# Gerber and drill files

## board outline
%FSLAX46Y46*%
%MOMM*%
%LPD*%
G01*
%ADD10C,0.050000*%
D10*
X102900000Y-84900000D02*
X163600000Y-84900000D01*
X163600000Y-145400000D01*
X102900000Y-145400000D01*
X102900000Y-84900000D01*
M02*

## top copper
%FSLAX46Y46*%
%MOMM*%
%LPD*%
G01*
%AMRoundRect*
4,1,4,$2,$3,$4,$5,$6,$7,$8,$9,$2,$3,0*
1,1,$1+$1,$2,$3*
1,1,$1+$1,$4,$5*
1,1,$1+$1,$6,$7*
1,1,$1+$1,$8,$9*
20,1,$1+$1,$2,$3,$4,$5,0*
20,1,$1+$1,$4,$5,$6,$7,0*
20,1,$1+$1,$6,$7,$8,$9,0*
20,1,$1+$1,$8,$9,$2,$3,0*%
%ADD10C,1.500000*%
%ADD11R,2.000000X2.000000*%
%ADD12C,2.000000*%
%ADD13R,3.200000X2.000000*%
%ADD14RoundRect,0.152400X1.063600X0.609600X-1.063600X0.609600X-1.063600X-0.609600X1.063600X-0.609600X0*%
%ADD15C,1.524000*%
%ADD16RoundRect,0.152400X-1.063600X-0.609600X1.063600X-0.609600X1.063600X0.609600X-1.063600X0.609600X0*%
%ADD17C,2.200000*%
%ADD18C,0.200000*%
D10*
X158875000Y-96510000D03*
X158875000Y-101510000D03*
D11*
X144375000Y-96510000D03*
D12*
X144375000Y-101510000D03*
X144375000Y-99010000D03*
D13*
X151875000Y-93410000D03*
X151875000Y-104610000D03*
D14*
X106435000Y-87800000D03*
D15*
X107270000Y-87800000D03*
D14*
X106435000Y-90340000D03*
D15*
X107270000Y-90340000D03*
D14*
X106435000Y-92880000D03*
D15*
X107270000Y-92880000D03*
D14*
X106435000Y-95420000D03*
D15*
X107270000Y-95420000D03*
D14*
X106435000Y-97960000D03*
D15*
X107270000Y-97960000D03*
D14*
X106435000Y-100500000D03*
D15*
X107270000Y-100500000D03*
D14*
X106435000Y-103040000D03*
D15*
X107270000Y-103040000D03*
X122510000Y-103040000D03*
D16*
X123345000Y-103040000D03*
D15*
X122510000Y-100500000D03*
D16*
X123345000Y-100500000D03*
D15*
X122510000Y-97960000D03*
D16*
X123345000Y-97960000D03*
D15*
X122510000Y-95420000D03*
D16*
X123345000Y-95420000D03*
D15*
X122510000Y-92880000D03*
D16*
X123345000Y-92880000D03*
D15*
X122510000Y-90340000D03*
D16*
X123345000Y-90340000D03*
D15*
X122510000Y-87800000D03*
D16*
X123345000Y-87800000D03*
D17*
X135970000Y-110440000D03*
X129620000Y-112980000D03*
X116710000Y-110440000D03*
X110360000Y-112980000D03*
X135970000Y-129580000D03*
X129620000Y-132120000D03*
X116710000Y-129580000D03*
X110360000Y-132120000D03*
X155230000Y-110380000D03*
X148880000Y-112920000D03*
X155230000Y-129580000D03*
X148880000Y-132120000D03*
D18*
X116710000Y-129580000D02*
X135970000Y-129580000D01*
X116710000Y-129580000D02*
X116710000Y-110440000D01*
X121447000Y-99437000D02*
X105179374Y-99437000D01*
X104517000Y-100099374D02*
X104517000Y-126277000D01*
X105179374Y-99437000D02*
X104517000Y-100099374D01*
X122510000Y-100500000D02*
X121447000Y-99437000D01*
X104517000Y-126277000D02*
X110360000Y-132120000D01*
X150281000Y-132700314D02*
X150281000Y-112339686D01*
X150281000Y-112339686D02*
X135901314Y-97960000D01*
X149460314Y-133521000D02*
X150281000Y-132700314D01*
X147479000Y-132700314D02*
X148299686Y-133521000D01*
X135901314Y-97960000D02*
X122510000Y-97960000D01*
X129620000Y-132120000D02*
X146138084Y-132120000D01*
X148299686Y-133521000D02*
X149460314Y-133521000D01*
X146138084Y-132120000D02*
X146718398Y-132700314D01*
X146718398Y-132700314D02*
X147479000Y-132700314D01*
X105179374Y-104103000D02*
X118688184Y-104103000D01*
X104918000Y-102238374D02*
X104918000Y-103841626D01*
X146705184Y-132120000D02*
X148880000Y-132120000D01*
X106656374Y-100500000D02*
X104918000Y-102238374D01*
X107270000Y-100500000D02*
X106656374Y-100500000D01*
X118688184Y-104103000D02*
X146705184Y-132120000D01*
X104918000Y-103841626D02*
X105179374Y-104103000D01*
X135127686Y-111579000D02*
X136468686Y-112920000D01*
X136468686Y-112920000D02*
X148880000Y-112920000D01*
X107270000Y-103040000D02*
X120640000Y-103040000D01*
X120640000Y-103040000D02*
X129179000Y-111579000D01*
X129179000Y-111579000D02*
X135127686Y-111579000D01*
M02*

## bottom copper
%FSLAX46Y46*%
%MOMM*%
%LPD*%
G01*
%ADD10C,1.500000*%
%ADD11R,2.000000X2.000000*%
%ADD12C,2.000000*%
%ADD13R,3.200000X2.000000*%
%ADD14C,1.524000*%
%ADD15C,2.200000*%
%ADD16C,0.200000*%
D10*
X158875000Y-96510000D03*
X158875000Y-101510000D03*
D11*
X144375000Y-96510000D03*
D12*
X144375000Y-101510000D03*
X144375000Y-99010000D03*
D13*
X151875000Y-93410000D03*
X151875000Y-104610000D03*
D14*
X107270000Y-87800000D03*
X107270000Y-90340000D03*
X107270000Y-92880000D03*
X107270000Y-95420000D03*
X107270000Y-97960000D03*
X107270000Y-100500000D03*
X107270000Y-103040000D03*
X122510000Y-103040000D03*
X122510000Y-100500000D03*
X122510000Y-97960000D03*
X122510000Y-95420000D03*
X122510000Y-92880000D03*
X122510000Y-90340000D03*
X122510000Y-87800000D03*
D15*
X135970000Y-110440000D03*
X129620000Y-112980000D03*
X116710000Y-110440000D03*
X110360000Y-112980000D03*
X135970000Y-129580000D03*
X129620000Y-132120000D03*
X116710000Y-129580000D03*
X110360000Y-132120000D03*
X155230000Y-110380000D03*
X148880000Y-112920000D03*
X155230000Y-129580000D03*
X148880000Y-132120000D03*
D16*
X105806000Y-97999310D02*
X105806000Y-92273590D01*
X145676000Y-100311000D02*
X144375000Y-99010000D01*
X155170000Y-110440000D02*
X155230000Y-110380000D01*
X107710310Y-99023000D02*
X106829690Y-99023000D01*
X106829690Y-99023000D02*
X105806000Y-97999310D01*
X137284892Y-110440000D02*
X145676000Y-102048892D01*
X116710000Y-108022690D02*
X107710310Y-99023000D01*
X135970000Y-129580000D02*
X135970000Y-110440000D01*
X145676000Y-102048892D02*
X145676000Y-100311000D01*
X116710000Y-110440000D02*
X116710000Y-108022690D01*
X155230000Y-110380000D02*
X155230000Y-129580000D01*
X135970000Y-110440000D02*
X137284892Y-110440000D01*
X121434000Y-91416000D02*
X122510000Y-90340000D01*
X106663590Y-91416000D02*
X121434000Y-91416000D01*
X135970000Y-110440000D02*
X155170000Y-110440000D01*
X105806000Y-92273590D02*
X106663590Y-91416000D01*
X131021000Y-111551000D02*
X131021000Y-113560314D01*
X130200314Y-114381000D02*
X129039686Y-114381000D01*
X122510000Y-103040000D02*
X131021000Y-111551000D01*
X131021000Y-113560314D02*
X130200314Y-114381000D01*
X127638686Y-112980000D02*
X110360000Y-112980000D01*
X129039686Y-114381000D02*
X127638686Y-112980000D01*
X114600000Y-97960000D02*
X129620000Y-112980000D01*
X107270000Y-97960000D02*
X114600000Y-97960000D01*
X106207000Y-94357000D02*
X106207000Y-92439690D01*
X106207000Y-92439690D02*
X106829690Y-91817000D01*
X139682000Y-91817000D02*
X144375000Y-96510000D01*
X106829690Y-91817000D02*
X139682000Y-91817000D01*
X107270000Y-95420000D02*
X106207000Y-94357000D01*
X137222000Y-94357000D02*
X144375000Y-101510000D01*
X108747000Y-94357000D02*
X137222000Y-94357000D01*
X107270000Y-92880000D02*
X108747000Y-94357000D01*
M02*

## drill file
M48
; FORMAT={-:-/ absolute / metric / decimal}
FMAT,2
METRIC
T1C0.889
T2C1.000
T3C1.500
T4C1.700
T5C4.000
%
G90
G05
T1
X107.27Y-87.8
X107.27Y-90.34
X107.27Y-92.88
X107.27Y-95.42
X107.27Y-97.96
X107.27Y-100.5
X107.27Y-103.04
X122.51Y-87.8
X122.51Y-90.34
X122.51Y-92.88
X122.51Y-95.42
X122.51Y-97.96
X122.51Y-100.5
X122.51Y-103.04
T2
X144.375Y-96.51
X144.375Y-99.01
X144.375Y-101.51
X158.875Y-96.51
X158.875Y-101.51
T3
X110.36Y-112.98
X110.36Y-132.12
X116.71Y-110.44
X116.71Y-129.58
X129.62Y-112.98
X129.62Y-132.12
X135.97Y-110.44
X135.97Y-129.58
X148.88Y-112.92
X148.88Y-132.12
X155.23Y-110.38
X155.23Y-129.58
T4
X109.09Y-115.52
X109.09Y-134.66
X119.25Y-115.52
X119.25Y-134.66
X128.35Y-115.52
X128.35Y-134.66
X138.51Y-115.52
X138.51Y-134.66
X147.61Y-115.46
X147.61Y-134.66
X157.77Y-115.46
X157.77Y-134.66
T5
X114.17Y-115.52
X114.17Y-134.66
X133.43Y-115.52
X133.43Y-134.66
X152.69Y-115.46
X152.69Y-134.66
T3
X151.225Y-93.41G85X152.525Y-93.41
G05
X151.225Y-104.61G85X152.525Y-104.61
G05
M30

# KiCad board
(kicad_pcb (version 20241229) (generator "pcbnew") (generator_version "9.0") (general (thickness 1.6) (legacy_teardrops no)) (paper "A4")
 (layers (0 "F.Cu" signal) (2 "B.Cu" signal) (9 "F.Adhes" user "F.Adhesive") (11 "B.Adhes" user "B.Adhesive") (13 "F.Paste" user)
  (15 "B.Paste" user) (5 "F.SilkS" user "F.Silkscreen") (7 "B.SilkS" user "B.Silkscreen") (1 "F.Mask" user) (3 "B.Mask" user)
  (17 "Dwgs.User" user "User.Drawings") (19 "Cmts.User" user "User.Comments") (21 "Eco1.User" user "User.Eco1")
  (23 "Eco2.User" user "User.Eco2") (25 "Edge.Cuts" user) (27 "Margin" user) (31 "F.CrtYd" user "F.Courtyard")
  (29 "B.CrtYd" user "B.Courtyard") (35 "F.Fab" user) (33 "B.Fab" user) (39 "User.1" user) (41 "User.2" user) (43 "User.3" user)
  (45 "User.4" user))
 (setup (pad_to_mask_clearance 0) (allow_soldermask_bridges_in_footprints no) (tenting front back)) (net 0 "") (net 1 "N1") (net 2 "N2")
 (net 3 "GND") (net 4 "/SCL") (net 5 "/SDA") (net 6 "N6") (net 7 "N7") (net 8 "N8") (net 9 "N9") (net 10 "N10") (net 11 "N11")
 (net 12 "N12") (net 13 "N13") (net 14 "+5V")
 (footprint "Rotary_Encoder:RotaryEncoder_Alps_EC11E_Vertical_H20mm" (layer "F.Cu") (at 144.375 96.51)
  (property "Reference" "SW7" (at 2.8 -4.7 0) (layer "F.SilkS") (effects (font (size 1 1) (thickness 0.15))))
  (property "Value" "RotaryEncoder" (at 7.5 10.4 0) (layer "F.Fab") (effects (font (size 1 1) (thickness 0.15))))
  (pad "" thru_hole circle (at 14.5 0) (size 1.5 1.5) (drill 1) (layers "*.Cu" "*.Mask") (remove_unused_layers no))
  (pad "" thru_hole circle (at 14.5 5) (size 1.5 1.5) (drill 1) (layers "*.Cu" "*.Mask") (remove_unused_layers no))
  (pad "A" thru_hole rect (at 0 0) (size 2 2) (drill 1) (layers "*.Cu" "*.Mask") (remove_unused_layers no) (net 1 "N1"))
  (pad "B" thru_hole circle (at 0 5) (size 2 2) (drill 1) (layers "*.Cu" "*.Mask") (remove_unused_layers no) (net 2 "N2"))
  (pad "C" thru_hole circle (at 0 2.5) (size 2 2) (drill 1) (layers "*.Cu" "*.Mask") (remove_unused_layers no) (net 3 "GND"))
  (pad "MP" thru_hole rect (at 7.5 -3.1) (size 3.2 2) (drill oval 2.8 1.5) (layers "*.Cu" "*.Mask") (remove_unused_layers no))
  (pad "MP" thru_hole rect (at 7.5 8.1) (size 3.2 2) (drill oval 2.8 1.5) (layers "*.Cu" "*.Mask") (remove_unused_layers no)))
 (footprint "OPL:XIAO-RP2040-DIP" (layer "F.Cu") (at 114.89 95.42)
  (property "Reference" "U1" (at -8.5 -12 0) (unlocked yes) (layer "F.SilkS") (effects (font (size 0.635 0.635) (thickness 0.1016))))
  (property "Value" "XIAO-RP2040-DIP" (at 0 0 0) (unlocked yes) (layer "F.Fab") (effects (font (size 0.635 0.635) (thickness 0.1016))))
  (pad "1" smd roundrect (at -8.455 -7.62 180) (size 2.432 1.524) (layers "F.Cu" "F.Mask") (roundrect_rratio 0.1) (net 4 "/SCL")
   (thermal_bridge_angle 45))
  (pad "1" thru_hole circle (at -7.62 -7.62 180) (size 1.524 1.524) (drill 0.889) (layers "*.Cu" "*.Mask") (remove_unused_layers no)
   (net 4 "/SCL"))
  (pad "2" smd roundrect (at -8.455 -5.08 180) (size 2.432 1.524) (layers "F.Cu" "F.Mask") (roundrect_rratio 0.1) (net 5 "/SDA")
   (thermal_bridge_angle 45))
  (pad "2" thru_hole circle (at -7.62 -5.08 180) (size 1.524 1.524) (drill 0.889) (layers "*.Cu" "*.Mask") (remove_unused_layers no)
   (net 5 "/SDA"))
  (pad "3" smd roundrect (at -8.455 -2.54 180) (size 2.432 1.524) (layers "F.Cu" "F.Mask") (roundrect_rratio 0.1) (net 2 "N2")
   (thermal_bridge_angle 45))
  (pad "3" thru_hole circle (at -7.62 -2.54 180) (size 1.524 1.524) (drill 0.889) (layers "*.Cu" "*.Mask") (remove_unused_layers no)
   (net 2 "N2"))
  (pad "4" smd roundrect (at -8.455 0 180) (size 2.432 1.524) (layers "F.Cu" "F.Mask") (roundrect_rratio 0.1) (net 1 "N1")
   (thermal_bridge_angle 45))
  (pad "4" thru_hole circle (at -7.62 0 180) (size 1.524 1.524) (drill 0.889) (layers "*.Cu" "*.Mask") (remove_unused_layers no)
   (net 1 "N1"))
  (pad "5" smd roundrect (at -8.455 2.54 180) (size 2.432 1.524) (layers "F.Cu" "F.Mask") (roundrect_rratio 0.1) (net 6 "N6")
   (thermal_bridge_angle 45))
  (pad "5" thru_hole circle (at -7.62 2.54 180) (size 1.524 1.524) (drill 0.889) (layers "*.Cu" "*.Mask") (remove_unused_layers no)
   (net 6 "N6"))
  (pad "6" smd roundrect (at -8.455 5.08 180) (size 2.432 1.524) (layers "F.Cu" "F.Mask") (roundrect_rratio 0.1) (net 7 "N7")
   (thermal_bridge_angle 45))
  (pad "6" thru_hole circle (at -7.62 5.08 180) (size 1.524 1.524) (drill 0.889) (layers "*.Cu" "*.Mask") (remove_unused_layers no)
   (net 7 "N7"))
  (pad "7" smd roundrect (at -8.455 7.62 180) (size 2.432 1.524) (layers "F.Cu" "F.Mask") (roundrect_rratio 0.1) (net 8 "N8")
   (thermal_bridge_angle 45))
  (pad "7" thru_hole circle (at -7.62 7.62 180) (size 1.524 1.524) (drill 0.889) (layers "*.Cu" "*.Mask") (remove_unused_layers no)
   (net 8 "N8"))
  (pad "8" thru_hole circle (at 7.62 7.62) (size 1.524 1.524) (drill 0.889) (layers "*.Cu" "*.Mask") (remove_unused_layers no) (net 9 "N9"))
  (pad "8" smd roundrect (at 8.455 7.62) (size 2.432 1.524) (layers "F.Cu" "F.Mask") (roundrect_rratio 0.1) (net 9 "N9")
   (thermal_bridge_angle 45))
  (pad "9" thru_hole circle (at 7.62 5.08) (size 1.524 1.524) (drill 0.889) (layers "*.Cu" "*.Mask") (remove_unused_layers no)
   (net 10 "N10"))
  (pad "9" smd roundrect (at 8.455 5.08) (size 2.432 1.524) (layers "F.Cu" "F.Mask") (roundrect_rratio 0.1) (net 10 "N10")
   (thermal_bridge_angle 45))
  (pad "10" thru_hole circle (at 7.62 2.54) (size 1.524 1.524) (drill 0.889) (layers "*.Cu" "*.Mask") (remove_unused_layers no)
   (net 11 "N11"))
  (pad "10" smd roundrect (at 8.455 2.54) (size 2.432 1.524) (layers "F.Cu" "F.Mask") (roundrect_rratio 0.1) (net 11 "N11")
   (thermal_bridge_angle 45))
  (pad "11" thru_hole circle (at 7.62 0) (size 1.524 1.524) (drill 0.889) (layers "*.Cu" "*.Mask") (remove_unused_layers no) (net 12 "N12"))
  (pad "11" smd roundrect (at 8.455 0) (size 2.432 1.524) (layers "F.Cu" "F.Mask") (roundrect_rratio 0.1) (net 12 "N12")
   (thermal_bridge_angle 45))
  (pad "12" thru_hole circle (at 7.62 -2.54) (size 1.524 1.524) (drill 0.889) (layers "*.Cu" "*.Mask") (remove_unused_layers no)
   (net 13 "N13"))
  (pad "12" smd roundrect (at 8.455 -2.54) (size 2.432 1.524) (layers "F.Cu" "F.Mask") (roundrect_rratio 0.1) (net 13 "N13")
   (thermal_bridge_angle 45))
  (pad "13" thru_hole circle (at 7.62 -5.08) (size 1.524 1.524) (drill 0.889) (layers "*.Cu" "*.Mask") (remove_unused_layers no)
   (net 3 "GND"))
  (pad "13" smd roundrect (at 8.455 -5.08) (size 2.432 1.524) (layers "F.Cu" "F.Mask") (roundrect_rratio 0.1) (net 3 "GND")
   (thermal_bridge_angle 45))
  (pad "14" thru_hole circle (at 7.62 -7.62) (size 1.524 1.524) (drill 0.889) (layers "*.Cu" "*.Mask") (remove_unused_layers no)
   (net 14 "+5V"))
  (pad "14" smd roundrect (at 8.455 -7.62) (size 2.432 1.524) (layers "F.Cu" "F.Mask") (roundrect_rratio 0.1) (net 14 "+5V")
   (thermal_bridge_angle 45)))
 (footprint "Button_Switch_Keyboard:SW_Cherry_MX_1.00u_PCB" (layer "F.Cu") (at 135.97 110.44)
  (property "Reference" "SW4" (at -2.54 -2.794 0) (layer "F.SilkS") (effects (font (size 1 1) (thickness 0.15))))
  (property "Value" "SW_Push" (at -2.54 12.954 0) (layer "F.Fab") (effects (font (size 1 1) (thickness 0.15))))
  (pad "" np_thru_hole circle (at -7.62 5.08) (size 1.7 1.7) (drill 1.7) (layers "*.Cu" "*.Mask"))
  (pad "" np_thru_hole circle (at -2.54 5.08) (size 4 4) (drill 4) (layers "*.Cu" "*.Mask"))
  (pad "" np_thru_hole circle (at 2.54 5.08) (size 1.7 1.7) (drill 1.7) (layers "*.Cu" "*.Mask"))
  (pad "1" thru_hole circle (at 0 0) (size 2.2 2.2) (drill 1.5) (layers "*.Cu" "*.Mask") (remove_unused_layers no) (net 3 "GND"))
  (pad "2" thru_hole circle (at -6.35 2.54) (size 2.2 2.2) (drill 1.5) (layers "*.Cu" "*.Mask") (remove_unused_layers no) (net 6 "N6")))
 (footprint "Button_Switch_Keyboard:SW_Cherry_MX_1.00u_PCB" (layer "F.Cu") (at 116.71 110.44)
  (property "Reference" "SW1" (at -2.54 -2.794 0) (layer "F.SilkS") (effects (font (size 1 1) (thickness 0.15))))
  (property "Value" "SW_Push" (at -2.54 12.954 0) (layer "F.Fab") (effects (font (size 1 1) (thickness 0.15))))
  (pad "" np_thru_hole circle (at -7.62 5.08) (size 1.7 1.7) (drill 1.7) (layers "*.Cu" "*.Mask"))
  (pad "" np_thru_hole circle (at -2.54 5.08) (size 4 4) (drill 4) (layers "*.Cu" "*.Mask"))
  (pad "" np_thru_hole circle (at 2.54 5.08) (size 1.7 1.7) (drill 1.7) (layers "*.Cu" "*.Mask"))
  (pad "1" thru_hole circle (at 0 0) (size 2.2 2.2) (drill 1.5) (layers "*.Cu" "*.Mask") (remove_unused_layers no) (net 3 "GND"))
  (pad "2" thru_hole circle (at -6.35 2.54) (size 2.2 2.2) (drill 1.5) (layers "*.Cu" "*.Mask") (remove_unused_layers no) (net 9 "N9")))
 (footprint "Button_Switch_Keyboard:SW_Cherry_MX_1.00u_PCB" (layer "F.Cu") (at 135.97 129.58)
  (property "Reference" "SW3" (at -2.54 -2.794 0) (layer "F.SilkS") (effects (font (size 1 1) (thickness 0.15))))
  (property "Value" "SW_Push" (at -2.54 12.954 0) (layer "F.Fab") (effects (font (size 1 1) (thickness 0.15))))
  (pad "" np_thru_hole circle (at -7.62 5.08) (size 1.7 1.7) (drill 1.7) (layers "*.Cu" "*.Mask"))
  (pad "" np_thru_hole circle (at -2.54 5.08) (size 4 4) (drill 4) (layers "*.Cu" "*.Mask"))
  (pad "" np_thru_hole circle (at 2.54 5.08) (size 1.7 1.7) (drill 1.7) (layers "*.Cu" "*.Mask"))
  (pad "1" thru_hole circle (at 0 0) (size 2.2 2.2) (drill 1.5) (layers "*.Cu" "*.Mask") (remove_unused_layers no) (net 3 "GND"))
  (pad "2" thru_hole circle (at -6.35 2.54) (size 2.2 2.2) (drill 1.5) (layers "*.Cu" "*.Mask") (remove_unused_layers no) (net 11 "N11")))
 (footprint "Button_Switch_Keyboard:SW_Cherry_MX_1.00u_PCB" (layer "F.Cu") (at 116.71 129.58)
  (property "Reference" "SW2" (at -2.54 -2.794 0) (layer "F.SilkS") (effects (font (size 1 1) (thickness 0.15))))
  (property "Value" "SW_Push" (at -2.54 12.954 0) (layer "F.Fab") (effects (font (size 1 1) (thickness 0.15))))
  (pad "" np_thru_hole circle (at -7.62 5.08) (size 1.7 1.7) (drill 1.7) (layers "*.Cu" "*.Mask"))
  (pad "" np_thru_hole circle (at -2.54 5.08) (size 4 4) (drill 4) (layers "*.Cu" "*.Mask"))
  (pad "" np_thru_hole circle (at 2.54 5.08) (size 1.7 1.7) (drill 1.7) (layers "*.Cu" "*.Mask"))
  (pad "1" thru_hole circle (at 0 0) (size 2.2 2.2) (drill 1.5) (layers "*.Cu" "*.Mask") (remove_unused_layers no) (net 3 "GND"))
  (pad "2" thru_hole circle (at -6.35 2.54) (size 2.2 2.2) (drill 1.5) (layers "*.Cu" "*.Mask") (remove_unused_layers no) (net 10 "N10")))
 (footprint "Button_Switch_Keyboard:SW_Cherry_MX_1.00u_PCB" (layer "F.Cu") (at 155.23 110.38)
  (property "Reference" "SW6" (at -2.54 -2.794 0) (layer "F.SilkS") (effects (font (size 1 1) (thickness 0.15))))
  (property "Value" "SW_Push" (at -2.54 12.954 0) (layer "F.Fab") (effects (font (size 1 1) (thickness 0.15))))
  (pad "" np_thru_hole circle (at -7.62 5.08) (size 1.7 1.7) (drill 1.7) (layers "*.Cu" "*.Mask"))
  (pad "" np_thru_hole circle (at -2.54 5.08) (size 4 4) (drill 4) (layers "*.Cu" "*.Mask"))
  (pad "" np_thru_hole circle (at 2.54 5.08) (size 1.7 1.7) (drill 1.7) (layers "*.Cu" "*.Mask"))
  (pad "1" thru_hole circle (at 0 0) (size 2.2 2.2) (drill 1.5) (layers "*.Cu" "*.Mask") (remove_unused_layers no) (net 3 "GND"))
  (pad "2" thru_hole circle (at -6.35 2.54) (size 2.2 2.2) (drill 1.5) (layers "*.Cu" "*.Mask") (remove_unused_layers no) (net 8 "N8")))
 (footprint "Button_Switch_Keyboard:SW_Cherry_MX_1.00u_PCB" (layer "F.Cu") (at 155.23 129.58)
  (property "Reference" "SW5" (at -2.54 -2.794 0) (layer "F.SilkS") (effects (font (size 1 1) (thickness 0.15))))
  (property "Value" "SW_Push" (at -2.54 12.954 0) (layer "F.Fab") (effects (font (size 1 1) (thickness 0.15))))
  (pad "" np_thru_hole circle (at -7.62 5.08) (size 1.7 1.7) (drill 1.7) (layers "*.Cu" "*.Mask"))
  (pad "" np_thru_hole circle (at -2.54 5.08) (size 4 4) (drill 4) (layers "*.Cu" "*.Mask"))
  (pad "" np_thru_hole circle (at 2.54 5.08) (size 1.7 1.7) (drill 1.7) (layers "*.Cu" "*.Mask"))
  (pad "1" thru_hole circle (at 0 0) (size 2.2 2.2) (drill 1.5) (layers "*.Cu" "*.Mask") (remove_unused_layers no) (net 3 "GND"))
  (pad "2" thru_hole circle (at -6.35 2.54) (size 2.2 2.2) (drill 1.5) (layers "*.Cu" "*.Mask") (remove_unused_layers no) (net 7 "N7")))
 (gr_rect (start 102.9 84.9) (end 163.6 145.4) (stroke (width 0.05) (type default)) (fill no) (layer "Edge.Cuts"))
 (segment (start 116.71 129.58) (end 135.97 129.58) (width 0.2) (layer "F.Cu") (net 3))
 (segment (start 116.71 129.58) (end 116.71 110.44) (width 0.2) (layer "F.Cu") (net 3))
 (segment (start 105.806 97.99931) (end 105.806 92.27359) (width 0.2) (layer "B.Cu") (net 3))
 (segment (start 145.676 100.311) (end 144.375 99.01) (width 0.2) (layer "B.Cu") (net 3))
 (segment (start 155.17 110.44) (end 155.23 110.38) (width 0.2) (layer "B.Cu") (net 3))
 (segment (start 107.71031 99.023) (end 106.82969 99.023) (width 0.2) (layer "B.Cu") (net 3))
 (segment (start 106.82969 99.023) (end 105.806 97.99931) (width 0.2) (layer "B.Cu") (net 3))
 (segment (start 137.284892 110.44) (end 145.676 102.048892) (width 0.2) (layer "B.Cu") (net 3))
 (segment (start 116.71 108.02269) (end 107.71031 99.023) (width 0.2) (layer "B.Cu") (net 3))
 (segment (start 135.97 129.58) (end 135.97 110.44) (width 0.2) (layer "B.Cu") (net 3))
 (segment (start 145.676 102.048892) (end 145.676 100.311) (width 0.2) (layer "B.Cu") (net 3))
 (segment (start 116.71 110.44) (end 116.71 108.02269) (width 0.2) (layer "B.Cu") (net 3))
 (segment (start 155.23 110.38) (end 155.23 129.58) (width 0.2) (layer "B.Cu") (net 3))
 (segment (start 135.97 110.44) (end 137.284892 110.44) (width 0.2) (layer "B.Cu") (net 3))
 (segment (start 121.434 91.416) (end 122.51 90.34) (width 0.2) (layer "B.Cu") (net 3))
 (segment (start 106.66359 91.416) (end 121.434 91.416) (width 0.2) (layer "B.Cu") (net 3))
 (segment (start 135.97 110.44) (end 155.17 110.44) (width 0.2) (layer "B.Cu") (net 3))
 (segment (start 105.806 92.27359) (end 106.66359 91.416) (width 0.2) (layer "B.Cu") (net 3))
 (segment (start 131.021 111.551) (end 131.021 113.560314) (width 0.2) (layer "B.Cu") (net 9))
 (segment (start 130.200314 114.381) (end 129.039686 114.381) (width 0.2) (layer "B.Cu") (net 9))
 (segment (start 122.51 103.04) (end 131.021 111.551) (width 0.2) (layer "B.Cu") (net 9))
 (segment (start 131.021 113.560314) (end 130.200314 114.381) (width 0.2) (layer "B.Cu") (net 9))
 (segment (start 127.638686 112.98) (end 110.36 112.98) (width 0.2) (layer "B.Cu") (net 9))
 (segment (start 129.039686 114.381) (end 127.638686 112.98) (width 0.2) (layer "B.Cu") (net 9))
 (segment (start 121.447 99.437) (end 105.179374 99.437) (width 0.2) (layer "F.Cu") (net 10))
 (segment (start 104.517 100.099374) (end 104.517 126.277) (width 0.2) (layer "F.Cu") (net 10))
 (segment (start 105.179374 99.437) (end 104.517 100.099374) (width 0.2) (layer "F.Cu") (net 10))
 (segment (start 122.51 100.5) (end 121.447 99.437) (width 0.2) (layer "F.Cu") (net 10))
 (segment (start 104.517 126.277) (end 110.36 132.12) (width 0.2) (layer "F.Cu") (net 10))
 (segment (start 150.281 132.700314) (end 150.281 112.339686) (width 0.2) (layer "F.Cu") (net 11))
 (segment (start 150.281 112.339686) (end 135.901314 97.96) (width 0.2) (layer "F.Cu") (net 11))
 (segment (start 149.460314 133.521) (end 150.281 132.700314) (width 0.2) (layer "F.Cu") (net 11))
 (segment (start 147.479 132.700314) (end 148.299686 133.521) (width 0.2) (layer "F.Cu") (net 11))
 (segment (start 135.901314 97.96) (end 122.51 97.96) (width 0.2) (layer "F.Cu") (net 11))
 (segment (start 129.62 132.12) (end 146.138084 132.12) (width 0.2) (layer "F.Cu") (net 11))
 (segment (start 148.299686 133.521) (end 149.460314 133.521) (width 0.2) (layer "F.Cu") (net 11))
 (segment (start 146.138084 132.12) (end 146.718398 132.700314) (width 0.2) (layer "F.Cu") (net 11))
 (segment (start 146.718398 132.700314) (end 147.479 132.700314) (width 0.2) (layer "F.Cu") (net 11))
 (segment (start 114.6 97.96) (end 129.62 112.98) (width 0.2) (layer "B.Cu") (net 6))
 (segment (start 107.27 97.96) (end 114.6 97.96) (width 0.2) (layer "B.Cu") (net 6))
 (segment (start 105.179374 104.103) (end 118.688184 104.103) (width 0.2) (layer "F.Cu") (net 7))
 (segment (start 104.918 102.238374) (end 104.918 103.841626) (width 0.2) (layer "F.Cu") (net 7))
 (segment (start 146.705184 132.12) (end 148.88 132.12) (width 0.2) (layer "F.Cu") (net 7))
 (segment (start 106.656374 100.5) (end 104.918 102.238374) (width 0.2) (layer "F.Cu") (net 7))
 (segment (start 107.27 100.5) (end 106.656374 100.5) (width 0.2) (layer "F.Cu") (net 7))
 (segment (start 118.688184 104.103) (end 146.705184 132.12) (width 0.2) (layer "F.Cu") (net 7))
 (segment (start 104.918 103.841626) (end 105.179374 104.103) (width 0.2) (layer "F.Cu") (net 7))
 (segment (start 135.127686 111.579) (end 136.468686 112.92) (width 0.2) (layer "F.Cu") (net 8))
 (segment (start 136.468686 112.92) (end 148.88 112.92) (width 0.2) (layer "F.Cu") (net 8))
 (segment (start 107.27 103.04) (end 120.64 103.04) (width 0.2) (layer "F.Cu") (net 8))
 (segment (start 120.64 103.04) (end 129.179 111.579) (width 0.2) (layer "F.Cu") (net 8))
 (segment (start 129.179 111.579) (end 135.127686 111.579) (width 0.2) (layer "F.Cu") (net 8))
 (segment (start 106.207 94.357) (end 106.207 92.43969) (width 0.2) (layer "B.Cu") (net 1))
 (segment (start 106.207 92.43969) (end 106.82969 91.817) (width 0.2) (layer "B.Cu") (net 1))
 (segment (start 139.682 91.817) (end 144.375 96.51) (width 0.2) (layer "B.Cu") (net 1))
 (segment (start 106.82969 91.817) (end 139.682 91.817) (width 0.2) (layer "B.Cu") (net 1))
 (segment (start 107.27 95.42) (end 106.207 94.357) (width 0.2) (layer "B.Cu") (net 1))
 (segment (start 137.222 94.357) (end 144.375 101.51) (width 0.2) (layer "B.Cu") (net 2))
 (segment (start 108.747 94.357) (end 137.222 94.357) (width 0.2) (layer "B.Cu") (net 2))
 (segment (start 107.27 92.88) (end 108.747 94.357) (width 0.2) (layer "B.Cu") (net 2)))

